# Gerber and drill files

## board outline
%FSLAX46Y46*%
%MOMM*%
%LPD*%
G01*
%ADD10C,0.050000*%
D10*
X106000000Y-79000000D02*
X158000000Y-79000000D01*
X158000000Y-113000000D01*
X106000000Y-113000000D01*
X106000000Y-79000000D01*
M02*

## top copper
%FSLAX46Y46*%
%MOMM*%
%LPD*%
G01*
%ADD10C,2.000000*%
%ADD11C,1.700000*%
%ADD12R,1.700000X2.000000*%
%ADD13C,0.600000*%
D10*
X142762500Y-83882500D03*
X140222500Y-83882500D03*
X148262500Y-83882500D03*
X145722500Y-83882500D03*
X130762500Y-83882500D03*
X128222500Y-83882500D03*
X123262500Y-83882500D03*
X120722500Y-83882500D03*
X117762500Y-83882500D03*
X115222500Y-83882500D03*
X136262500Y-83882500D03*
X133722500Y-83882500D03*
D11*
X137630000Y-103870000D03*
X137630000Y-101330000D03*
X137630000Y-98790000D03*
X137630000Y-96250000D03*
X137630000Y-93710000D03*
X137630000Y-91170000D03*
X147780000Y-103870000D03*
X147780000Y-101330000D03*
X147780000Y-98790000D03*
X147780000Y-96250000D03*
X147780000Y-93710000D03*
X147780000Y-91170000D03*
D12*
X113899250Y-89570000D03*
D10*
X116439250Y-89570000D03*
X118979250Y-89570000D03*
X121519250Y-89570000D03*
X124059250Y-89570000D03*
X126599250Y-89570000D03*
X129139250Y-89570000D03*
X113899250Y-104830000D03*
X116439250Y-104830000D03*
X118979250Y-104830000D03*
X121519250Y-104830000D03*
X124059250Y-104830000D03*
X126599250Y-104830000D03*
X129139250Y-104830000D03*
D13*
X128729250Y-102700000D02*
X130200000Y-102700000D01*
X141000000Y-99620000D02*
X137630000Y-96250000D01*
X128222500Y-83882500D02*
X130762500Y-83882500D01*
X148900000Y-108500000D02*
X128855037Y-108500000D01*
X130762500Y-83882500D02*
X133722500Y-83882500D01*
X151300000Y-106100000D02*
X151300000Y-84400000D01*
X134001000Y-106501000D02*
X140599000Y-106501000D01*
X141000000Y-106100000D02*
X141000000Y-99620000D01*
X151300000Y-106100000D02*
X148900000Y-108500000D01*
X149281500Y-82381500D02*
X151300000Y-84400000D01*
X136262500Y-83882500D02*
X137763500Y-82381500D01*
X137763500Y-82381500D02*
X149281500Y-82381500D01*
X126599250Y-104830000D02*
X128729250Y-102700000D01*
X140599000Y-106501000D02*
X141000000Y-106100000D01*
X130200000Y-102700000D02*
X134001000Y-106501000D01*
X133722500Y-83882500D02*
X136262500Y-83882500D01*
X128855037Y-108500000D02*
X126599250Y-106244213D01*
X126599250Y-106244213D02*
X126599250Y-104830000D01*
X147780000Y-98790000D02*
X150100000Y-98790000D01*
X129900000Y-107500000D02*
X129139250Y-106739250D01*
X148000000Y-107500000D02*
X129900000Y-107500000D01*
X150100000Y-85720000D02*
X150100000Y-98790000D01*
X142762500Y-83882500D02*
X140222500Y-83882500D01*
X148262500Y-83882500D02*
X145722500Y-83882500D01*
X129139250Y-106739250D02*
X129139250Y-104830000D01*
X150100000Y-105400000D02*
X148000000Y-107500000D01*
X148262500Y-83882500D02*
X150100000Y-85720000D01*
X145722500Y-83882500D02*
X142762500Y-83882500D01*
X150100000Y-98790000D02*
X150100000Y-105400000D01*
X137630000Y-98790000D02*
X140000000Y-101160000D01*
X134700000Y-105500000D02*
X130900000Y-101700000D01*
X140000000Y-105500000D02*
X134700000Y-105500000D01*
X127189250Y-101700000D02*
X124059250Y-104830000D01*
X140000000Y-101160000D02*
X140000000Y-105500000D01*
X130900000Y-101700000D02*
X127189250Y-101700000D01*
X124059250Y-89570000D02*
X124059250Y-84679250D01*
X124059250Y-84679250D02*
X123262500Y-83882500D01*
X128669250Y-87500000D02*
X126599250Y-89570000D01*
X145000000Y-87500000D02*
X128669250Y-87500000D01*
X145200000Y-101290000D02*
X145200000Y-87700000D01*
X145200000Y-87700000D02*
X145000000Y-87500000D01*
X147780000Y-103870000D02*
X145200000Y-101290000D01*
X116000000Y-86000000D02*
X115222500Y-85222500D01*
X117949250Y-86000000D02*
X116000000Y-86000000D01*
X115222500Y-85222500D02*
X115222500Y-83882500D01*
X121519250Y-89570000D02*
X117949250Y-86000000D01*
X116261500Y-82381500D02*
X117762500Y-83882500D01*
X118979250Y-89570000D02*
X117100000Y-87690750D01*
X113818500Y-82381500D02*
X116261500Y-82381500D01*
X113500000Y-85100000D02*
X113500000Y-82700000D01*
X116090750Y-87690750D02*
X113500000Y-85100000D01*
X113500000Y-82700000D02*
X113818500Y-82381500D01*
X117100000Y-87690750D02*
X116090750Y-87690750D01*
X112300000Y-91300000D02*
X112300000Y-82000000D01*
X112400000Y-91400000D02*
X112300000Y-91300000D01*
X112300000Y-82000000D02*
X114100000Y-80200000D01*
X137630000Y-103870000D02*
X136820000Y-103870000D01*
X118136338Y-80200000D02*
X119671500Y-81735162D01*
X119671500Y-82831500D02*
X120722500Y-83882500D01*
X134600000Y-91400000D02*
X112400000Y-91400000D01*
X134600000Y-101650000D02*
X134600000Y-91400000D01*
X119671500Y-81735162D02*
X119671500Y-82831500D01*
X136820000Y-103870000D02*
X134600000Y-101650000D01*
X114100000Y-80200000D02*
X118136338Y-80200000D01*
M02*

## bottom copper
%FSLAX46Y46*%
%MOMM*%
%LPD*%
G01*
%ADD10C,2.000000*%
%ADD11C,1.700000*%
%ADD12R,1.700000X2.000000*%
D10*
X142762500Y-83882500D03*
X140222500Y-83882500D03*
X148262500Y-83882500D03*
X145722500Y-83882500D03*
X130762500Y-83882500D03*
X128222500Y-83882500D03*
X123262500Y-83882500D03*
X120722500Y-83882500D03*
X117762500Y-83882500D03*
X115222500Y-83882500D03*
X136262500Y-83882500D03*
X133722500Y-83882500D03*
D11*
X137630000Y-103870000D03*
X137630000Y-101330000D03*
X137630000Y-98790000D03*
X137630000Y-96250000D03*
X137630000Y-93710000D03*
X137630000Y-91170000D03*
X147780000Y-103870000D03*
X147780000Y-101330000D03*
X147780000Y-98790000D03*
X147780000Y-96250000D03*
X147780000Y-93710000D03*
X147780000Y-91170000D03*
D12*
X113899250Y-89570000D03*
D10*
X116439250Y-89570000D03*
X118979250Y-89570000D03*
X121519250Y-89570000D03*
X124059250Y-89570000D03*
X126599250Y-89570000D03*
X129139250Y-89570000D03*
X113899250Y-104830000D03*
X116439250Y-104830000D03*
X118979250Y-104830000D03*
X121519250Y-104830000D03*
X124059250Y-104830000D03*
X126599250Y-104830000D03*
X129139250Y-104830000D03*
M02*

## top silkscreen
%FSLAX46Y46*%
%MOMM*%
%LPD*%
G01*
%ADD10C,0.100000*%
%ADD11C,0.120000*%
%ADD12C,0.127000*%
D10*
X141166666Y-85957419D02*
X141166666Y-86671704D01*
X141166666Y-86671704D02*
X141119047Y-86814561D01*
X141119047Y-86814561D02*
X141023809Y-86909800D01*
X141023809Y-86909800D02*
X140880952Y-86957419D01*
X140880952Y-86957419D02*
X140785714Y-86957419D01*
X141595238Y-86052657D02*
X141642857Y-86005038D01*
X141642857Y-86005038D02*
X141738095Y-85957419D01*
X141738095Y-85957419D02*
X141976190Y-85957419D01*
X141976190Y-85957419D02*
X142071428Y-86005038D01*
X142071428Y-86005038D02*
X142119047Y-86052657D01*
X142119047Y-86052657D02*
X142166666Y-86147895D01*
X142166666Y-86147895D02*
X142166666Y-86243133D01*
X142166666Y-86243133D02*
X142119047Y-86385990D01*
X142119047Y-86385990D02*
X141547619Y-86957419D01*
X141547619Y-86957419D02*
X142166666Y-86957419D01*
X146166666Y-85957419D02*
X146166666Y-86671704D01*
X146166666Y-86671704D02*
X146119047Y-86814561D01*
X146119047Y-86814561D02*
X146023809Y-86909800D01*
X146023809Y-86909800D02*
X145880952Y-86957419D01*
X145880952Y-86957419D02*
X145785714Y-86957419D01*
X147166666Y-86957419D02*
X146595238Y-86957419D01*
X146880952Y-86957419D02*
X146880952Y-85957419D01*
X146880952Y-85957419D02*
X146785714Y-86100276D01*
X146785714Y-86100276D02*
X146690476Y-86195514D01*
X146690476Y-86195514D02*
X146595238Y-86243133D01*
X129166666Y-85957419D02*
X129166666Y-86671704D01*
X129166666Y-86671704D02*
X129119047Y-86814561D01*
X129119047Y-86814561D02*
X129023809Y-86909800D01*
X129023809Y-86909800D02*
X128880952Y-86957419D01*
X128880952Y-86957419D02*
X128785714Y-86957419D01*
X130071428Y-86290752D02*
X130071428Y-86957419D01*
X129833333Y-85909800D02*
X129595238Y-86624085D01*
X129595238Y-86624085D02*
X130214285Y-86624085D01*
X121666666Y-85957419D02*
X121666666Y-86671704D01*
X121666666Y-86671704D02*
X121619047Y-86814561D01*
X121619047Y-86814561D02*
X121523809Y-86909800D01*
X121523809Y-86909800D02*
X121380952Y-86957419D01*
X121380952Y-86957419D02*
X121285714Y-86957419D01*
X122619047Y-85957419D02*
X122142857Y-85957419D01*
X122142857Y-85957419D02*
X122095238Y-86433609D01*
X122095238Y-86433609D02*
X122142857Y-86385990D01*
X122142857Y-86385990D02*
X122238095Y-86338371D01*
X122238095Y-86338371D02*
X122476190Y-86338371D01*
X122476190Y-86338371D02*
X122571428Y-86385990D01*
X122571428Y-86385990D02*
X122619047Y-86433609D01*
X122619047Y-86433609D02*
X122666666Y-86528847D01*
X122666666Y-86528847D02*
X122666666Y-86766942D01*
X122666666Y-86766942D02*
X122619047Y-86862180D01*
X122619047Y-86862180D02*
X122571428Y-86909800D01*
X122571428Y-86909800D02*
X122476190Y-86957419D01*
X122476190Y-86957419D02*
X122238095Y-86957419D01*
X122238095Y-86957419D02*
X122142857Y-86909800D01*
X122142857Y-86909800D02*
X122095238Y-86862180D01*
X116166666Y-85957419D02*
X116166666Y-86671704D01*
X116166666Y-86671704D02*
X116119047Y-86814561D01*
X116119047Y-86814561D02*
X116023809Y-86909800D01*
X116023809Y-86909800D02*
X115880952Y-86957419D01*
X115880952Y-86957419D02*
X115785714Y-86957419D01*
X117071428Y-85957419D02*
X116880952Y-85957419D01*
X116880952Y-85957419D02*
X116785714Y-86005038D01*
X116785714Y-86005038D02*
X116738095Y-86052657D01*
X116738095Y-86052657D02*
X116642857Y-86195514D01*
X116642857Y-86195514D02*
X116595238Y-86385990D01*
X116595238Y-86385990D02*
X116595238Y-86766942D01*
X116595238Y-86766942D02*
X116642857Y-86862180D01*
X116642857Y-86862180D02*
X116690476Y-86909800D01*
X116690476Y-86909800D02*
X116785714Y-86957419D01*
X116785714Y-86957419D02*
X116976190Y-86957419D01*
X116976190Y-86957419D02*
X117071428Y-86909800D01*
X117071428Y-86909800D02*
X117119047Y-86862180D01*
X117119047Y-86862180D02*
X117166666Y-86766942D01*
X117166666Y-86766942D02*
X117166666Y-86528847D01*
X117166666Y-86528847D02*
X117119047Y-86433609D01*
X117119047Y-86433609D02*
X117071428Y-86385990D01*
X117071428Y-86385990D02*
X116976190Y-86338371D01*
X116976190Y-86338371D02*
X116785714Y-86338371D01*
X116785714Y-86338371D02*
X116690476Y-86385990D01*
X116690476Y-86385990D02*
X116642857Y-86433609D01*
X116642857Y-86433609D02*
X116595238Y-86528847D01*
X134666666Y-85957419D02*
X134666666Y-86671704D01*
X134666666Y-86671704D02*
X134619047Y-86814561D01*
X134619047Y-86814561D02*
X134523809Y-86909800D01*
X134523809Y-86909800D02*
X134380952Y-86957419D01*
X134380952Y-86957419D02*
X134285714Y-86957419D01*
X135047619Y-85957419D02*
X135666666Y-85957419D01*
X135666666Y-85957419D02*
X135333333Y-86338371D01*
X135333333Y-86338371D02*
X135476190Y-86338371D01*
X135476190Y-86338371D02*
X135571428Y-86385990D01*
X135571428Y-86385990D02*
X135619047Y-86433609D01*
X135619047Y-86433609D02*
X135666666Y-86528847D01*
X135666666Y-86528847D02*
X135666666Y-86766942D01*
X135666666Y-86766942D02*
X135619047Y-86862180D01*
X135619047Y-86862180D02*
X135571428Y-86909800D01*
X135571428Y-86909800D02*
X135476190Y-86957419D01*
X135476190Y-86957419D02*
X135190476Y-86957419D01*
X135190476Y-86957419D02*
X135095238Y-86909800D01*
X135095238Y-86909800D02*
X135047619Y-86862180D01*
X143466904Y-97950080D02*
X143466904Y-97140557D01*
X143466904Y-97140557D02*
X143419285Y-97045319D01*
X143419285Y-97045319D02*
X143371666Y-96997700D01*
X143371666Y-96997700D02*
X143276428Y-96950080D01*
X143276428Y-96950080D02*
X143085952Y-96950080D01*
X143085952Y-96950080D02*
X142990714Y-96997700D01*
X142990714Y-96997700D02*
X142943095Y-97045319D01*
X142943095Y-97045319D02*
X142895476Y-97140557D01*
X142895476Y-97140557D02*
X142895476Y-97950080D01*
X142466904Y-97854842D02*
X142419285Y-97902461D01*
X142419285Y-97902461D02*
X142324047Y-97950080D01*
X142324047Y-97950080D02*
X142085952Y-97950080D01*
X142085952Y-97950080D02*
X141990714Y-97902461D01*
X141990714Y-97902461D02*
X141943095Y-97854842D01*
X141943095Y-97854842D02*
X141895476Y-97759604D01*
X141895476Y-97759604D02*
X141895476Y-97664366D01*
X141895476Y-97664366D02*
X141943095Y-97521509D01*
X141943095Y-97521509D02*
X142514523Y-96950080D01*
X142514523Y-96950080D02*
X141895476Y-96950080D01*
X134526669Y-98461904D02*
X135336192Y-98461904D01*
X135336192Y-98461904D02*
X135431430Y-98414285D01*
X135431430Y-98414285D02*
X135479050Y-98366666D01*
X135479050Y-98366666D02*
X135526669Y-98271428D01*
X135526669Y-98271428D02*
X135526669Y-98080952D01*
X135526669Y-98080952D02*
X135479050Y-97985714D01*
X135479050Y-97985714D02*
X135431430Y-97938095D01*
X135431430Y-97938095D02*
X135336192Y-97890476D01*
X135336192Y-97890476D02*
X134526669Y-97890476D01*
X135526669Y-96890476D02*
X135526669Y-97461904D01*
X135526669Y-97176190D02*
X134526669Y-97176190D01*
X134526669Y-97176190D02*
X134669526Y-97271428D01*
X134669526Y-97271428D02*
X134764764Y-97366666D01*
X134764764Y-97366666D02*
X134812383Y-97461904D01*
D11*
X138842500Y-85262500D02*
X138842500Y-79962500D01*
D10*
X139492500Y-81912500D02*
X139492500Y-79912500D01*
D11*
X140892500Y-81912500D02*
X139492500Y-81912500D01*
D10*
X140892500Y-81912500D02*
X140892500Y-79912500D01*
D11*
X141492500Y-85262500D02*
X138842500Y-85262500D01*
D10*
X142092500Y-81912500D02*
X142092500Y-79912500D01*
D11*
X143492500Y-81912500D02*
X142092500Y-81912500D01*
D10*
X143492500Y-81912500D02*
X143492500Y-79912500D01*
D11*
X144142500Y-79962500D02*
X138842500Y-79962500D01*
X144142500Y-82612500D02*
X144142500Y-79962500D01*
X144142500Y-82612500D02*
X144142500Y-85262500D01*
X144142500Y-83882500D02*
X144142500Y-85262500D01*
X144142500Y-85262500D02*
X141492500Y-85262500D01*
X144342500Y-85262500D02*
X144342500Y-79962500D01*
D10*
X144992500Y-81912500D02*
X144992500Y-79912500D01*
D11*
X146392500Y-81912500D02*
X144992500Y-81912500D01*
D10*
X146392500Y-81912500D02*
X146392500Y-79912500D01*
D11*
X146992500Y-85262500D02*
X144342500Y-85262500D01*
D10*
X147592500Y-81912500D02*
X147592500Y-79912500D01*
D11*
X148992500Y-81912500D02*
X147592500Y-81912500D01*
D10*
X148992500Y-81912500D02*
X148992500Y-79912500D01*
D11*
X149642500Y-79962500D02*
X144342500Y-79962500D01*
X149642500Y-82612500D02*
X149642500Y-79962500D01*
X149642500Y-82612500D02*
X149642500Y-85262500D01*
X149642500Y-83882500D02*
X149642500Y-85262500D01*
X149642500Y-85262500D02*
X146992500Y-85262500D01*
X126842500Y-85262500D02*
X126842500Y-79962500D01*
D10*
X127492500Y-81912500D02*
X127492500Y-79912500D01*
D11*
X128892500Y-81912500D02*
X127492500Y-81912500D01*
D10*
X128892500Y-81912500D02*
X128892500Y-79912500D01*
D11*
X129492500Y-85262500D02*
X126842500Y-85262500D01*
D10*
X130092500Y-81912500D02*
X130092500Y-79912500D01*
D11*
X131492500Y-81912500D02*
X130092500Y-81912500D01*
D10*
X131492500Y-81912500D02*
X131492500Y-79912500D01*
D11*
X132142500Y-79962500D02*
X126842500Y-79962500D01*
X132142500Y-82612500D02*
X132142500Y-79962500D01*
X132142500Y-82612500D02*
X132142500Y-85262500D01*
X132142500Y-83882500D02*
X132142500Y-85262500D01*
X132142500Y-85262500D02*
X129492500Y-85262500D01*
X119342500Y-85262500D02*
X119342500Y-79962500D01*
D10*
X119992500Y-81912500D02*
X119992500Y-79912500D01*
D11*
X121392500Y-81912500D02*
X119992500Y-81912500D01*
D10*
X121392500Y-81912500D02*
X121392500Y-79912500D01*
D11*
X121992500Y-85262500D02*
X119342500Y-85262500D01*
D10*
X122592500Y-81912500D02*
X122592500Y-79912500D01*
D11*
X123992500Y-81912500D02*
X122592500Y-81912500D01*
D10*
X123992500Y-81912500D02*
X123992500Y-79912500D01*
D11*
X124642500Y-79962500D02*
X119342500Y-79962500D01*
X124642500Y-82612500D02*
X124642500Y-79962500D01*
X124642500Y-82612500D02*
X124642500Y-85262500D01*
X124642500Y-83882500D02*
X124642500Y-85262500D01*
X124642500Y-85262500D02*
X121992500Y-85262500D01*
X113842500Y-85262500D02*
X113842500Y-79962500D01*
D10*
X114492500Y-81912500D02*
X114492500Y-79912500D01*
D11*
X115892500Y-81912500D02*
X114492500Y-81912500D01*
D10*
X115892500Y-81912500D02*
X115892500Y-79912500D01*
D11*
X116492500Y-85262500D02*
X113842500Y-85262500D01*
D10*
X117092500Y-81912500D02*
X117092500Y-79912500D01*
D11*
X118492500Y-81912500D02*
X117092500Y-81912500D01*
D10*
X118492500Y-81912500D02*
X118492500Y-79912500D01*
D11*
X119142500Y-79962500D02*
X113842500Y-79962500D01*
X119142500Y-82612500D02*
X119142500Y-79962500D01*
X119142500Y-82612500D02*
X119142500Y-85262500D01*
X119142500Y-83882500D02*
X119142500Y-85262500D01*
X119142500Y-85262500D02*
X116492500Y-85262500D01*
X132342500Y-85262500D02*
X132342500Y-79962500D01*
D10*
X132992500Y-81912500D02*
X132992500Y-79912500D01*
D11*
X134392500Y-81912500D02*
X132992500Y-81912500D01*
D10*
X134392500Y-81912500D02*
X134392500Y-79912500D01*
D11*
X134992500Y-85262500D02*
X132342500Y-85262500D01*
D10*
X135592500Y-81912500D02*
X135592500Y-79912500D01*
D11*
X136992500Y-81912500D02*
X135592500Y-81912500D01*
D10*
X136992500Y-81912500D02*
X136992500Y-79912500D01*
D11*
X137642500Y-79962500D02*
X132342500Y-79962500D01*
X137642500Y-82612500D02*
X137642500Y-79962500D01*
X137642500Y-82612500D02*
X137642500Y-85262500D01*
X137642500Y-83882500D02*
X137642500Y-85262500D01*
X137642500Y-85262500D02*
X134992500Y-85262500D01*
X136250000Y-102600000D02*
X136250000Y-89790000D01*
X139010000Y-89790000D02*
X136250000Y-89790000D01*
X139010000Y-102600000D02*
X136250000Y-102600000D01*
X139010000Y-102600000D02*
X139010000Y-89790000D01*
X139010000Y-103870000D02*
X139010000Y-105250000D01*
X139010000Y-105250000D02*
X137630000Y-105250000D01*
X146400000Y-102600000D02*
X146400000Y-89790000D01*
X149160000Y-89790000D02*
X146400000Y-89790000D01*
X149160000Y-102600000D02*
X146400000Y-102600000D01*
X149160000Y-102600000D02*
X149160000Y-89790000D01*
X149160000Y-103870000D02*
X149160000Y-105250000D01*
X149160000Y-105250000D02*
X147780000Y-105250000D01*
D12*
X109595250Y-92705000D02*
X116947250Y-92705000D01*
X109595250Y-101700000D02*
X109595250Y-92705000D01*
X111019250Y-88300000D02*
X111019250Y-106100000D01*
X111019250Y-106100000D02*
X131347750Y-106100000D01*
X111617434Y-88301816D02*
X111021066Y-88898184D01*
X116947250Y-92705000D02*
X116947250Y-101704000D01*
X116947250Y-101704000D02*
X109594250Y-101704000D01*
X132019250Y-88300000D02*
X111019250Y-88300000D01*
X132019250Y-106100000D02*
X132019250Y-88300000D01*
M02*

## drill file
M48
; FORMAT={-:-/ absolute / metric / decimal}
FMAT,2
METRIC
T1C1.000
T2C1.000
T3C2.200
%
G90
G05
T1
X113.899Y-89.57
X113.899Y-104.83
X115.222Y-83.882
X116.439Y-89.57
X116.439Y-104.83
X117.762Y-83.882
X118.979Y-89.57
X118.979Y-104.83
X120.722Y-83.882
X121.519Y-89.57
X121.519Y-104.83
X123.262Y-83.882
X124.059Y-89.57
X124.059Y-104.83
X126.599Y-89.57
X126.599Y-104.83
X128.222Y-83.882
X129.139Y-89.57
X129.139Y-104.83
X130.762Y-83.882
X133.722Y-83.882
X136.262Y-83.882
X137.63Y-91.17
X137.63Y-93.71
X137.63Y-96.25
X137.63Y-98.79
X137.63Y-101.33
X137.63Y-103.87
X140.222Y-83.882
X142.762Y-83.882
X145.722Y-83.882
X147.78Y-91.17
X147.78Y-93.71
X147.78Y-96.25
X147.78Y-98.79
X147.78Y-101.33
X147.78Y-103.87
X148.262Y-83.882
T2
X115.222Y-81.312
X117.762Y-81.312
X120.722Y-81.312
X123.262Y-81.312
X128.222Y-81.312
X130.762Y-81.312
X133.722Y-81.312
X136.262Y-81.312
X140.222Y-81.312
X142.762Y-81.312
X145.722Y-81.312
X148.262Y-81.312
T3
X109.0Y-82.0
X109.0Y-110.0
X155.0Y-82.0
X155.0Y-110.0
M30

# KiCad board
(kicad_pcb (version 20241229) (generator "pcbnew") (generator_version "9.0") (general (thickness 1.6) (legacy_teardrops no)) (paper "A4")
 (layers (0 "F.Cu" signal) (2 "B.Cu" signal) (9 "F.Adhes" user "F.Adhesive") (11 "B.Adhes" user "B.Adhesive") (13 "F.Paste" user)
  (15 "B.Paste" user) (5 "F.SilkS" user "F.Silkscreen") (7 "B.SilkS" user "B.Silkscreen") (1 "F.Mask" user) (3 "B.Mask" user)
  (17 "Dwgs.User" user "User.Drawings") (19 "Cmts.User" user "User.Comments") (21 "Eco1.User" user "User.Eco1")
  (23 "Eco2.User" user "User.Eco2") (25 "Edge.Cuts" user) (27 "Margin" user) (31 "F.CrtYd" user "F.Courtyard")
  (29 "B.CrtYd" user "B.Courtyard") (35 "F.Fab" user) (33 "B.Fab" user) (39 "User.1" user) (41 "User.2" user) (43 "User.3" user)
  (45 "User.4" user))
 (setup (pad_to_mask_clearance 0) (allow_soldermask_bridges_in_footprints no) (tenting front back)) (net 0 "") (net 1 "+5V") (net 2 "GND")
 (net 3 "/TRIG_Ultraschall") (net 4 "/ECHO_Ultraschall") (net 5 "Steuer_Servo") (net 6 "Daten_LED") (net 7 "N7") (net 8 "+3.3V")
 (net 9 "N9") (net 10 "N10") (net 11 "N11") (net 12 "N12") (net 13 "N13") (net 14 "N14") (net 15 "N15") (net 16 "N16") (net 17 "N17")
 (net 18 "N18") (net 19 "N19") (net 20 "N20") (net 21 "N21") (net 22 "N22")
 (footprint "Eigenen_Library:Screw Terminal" (layer "F.Cu") (at 141.4925 79.9125 180)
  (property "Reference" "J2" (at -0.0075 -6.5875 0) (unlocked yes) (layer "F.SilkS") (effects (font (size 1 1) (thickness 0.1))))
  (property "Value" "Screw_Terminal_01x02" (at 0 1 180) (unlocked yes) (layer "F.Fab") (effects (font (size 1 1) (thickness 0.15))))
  (fp_line (start 2.65 -5.35) (end 2.65 -0.05) (stroke (width 0.12) (type solid)) (layer "F.SilkS"))
  (fp_line (start 2 -2) (end 2 0) (stroke (width 0.1) (type default)) (layer "F.SilkS"))
  (fp_line (start 0.6 -2) (end 2 -2) (stroke (width 0.12) (type solid)) (layer "F.SilkS"))
  (fp_line (start 0.6 -2) (end 0.6 0) (stroke (width 0.1) (type default)) (layer "F.SilkS"))
  (fp_line (start 0 -5.35) (end 2.65 -5.35) (stroke (width 0.12) (type solid)) (layer "F.SilkS"))
  (fp_line (start -0.6 -2) (end -0.6 0) (stroke (width 0.1) (type default)) (layer "F.SilkS"))
  (fp_line (start -2 -2) (end -0.6 -2) (stroke (width 0.12) (type solid)) (layer "F.SilkS"))
  (fp_line (start -2 -2) (end -2 0) (stroke (width 0.1) (type default)) (layer "F.SilkS"))
  (fp_line (start -2.65 -0.05) (end 2.65 -0.05) (stroke (width 0.12) (type solid)) (layer "F.SilkS"))
  (fp_line (start -2.65 -2.7) (end -2.65 -0.05) (stroke (width 0.12) (type solid)) (layer "F.SilkS"))
  (fp_line (start -2.65 -2.7) (end -2.65 -5.35) (stroke (width 0.12) (type solid)) (layer "F.SilkS"))
  (fp_line (start -2.65 -3.97) (end -2.65 -5.35) (stroke (width 0.12) (type solid)) (layer "F.SilkS"))
  (fp_line (start -2.65 -5.35) (end 0 -5.35) (stroke (width 0.12) (type solid)) (layer "F.SilkS"))
  (pad "" np_thru_hole circle (at -1.27 -1.4 270) (size 1 1) (drill 1) (layers "*.Mask"))
  (pad "" np_thru_hole circle (at 1.27 -1.4 180) (size 1 1) (drill 1) (layers "*.Mask"))
  (pad "1" thru_hole circle (at -1.27 -3.97 180) (size 2 2) (drill 1) (layers "*.Cu" "*.Mask") (remove_unused_layers no) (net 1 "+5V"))
  (pad "2" thru_hole circle (at 1.27 -3.97 180) (size 2 2) (drill 1) (layers "*.Cu" "*.Mask") (remove_unused_layers no) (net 1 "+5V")))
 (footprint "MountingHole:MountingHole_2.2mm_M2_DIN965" (layer "F.Cu") (at 155 110)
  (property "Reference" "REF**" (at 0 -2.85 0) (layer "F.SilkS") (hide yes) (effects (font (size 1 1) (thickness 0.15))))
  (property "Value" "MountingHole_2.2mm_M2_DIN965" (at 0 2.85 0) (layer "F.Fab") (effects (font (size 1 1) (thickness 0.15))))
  (pad "" np_thru_hole circle (at 0 0) (size 2.2 2.2) (drill 2.2) (layers "*.Cu" "*.Mask")))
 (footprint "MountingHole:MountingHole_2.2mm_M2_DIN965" (layer "F.Cu") (at 155 82)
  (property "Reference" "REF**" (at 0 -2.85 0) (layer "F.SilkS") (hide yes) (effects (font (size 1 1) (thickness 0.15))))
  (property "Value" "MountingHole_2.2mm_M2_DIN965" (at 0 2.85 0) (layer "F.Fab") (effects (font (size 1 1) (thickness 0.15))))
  (pad "" np_thru_hole circle (at 0 0) (size 2.2 2.2) (drill 2.2) (layers "*.Cu" "*.Mask")))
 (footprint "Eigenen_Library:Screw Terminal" (layer "F.Cu") (at 146.9925 79.9125 180)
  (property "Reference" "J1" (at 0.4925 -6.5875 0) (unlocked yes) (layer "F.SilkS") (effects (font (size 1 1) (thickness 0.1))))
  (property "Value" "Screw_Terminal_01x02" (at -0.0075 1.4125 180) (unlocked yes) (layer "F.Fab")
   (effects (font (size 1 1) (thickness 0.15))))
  (fp_line (start 2.65 -5.35) (end 2.65 -0.05) (stroke (width 0.12) (type solid)) (layer "F.SilkS"))
  (fp_line (start 2 -2) (end 2 0) (stroke (width 0.1) (type default)) (layer "F.SilkS"))
  (fp_line (start 0.6 -2) (end 2 -2) (stroke (width 0.12) (type solid)) (layer "F.SilkS"))
  (fp_line (start 0.6 -2) (end 0.6 0) (stroke (width 0.1) (type default)) (layer "F.SilkS"))
  (fp_line (start 0 -5.35) (end 2.65 -5.35) (stroke (width 0.12) (type solid)) (layer "F.SilkS"))
  (fp_line (start -0.6 -2) (end -0.6 0) (stroke (width 0.1) (type default)) (layer "F.SilkS"))
  (fp_line (start -2 -2) (end -0.6 -2) (stroke (width 0.12) (type solid)) (layer "F.SilkS"))
  (fp_line (start -2 -2) (end -2 0) (stroke (width 0.1) (type default)) (layer "F.SilkS"))
  (fp_line (start -2.65 -0.05) (end 2.65 -0.05) (stroke (width 0.12) (type solid)) (layer "F.SilkS"))
  (fp_line (start -2.65 -2.7) (end -2.65 -0.05) (stroke (width 0.12) (type solid)) (layer "F.SilkS"))
  (fp_line (start -2.65 -2.7) (end -2.65 -5.35) (stroke (width 0.12) (type solid)) (layer "F.SilkS"))
  (fp_line (start -2.65 -3.97) (end -2.65 -5.35) (stroke (width 0.12) (type solid)) (layer "F.SilkS"))
  (fp_line (start -2.65 -5.35) (end 0 -5.35) (stroke (width 0.12) (type solid)) (layer "F.SilkS"))
  (pad "" np_thru_hole circle (at -1.27 -1.4 270) (size 1 1) (drill 1) (layers "*.Mask"))
  (pad "" np_thru_hole circle (at 1.27 -1.4 180) (size 1 1) (drill 1) (layers "*.Mask"))
  (pad "1" thru_hole circle (at -1.27 -3.97 180) (size 2 2) (drill 1) (layers "*.Cu" "*.Mask") (remove_unused_layers no) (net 1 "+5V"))
  (pad "2" thru_hole circle (at 1.27 -3.97 180) (size 2 2) (drill 1) (layers "*.Cu" "*.Mask") (remove_unused_layers no) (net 1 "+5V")))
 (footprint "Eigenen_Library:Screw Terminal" (layer "F.Cu") (at 129.4925 79.9125 180)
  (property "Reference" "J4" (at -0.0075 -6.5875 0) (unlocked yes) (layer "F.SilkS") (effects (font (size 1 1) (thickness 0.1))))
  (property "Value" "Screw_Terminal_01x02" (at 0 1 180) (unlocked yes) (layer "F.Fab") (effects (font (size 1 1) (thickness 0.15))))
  (fp_line (start 2.65 -5.35) (end 2.65 -0.05) (stroke (width 0.12) (type solid)) (layer "F.SilkS"))
  (fp_line (start 2 -2) (end 2 0) (stroke (width 0.1) (type default)) (layer "F.SilkS"))
  (fp_line (start 0.6 -2) (end 2 -2) (stroke (width 0.12) (type solid)) (layer "F.SilkS"))
  (fp_line (start 0.6 -2) (end 0.6 0) (stroke (width 0.1) (type default)) (layer "F.SilkS"))
  (fp_line (start 0 -5.35) (end 2.65 -5.35) (stroke (width 0.12) (type solid)) (layer "F.SilkS"))
  (fp_line (start -0.6 -2) (end -0.6 0) (stroke (width 0.1) (type default)) (layer "F.SilkS"))
  (fp_line (start -2 -2) (end -0.6 -2) (stroke (width 0.12) (type solid)) (layer "F.SilkS"))
  (fp_line (start -2 -2) (end -2 0) (stroke (width 0.1) (type default)) (layer "F.SilkS"))
  (fp_line (start -2.65 -0.05) (end 2.65 -0.05) (stroke (width 0.12) (type solid)) (layer "F.SilkS"))
  (fp_line (start -2.65 -2.7) (end -2.65 -0.05) (stroke (width 0.12) (type solid)) (layer "F.SilkS"))
  (fp_line (start -2.65 -2.7) (end -2.65 -5.35) (stroke (width 0.12) (type solid)) (layer "F.SilkS"))
  (fp_line (start -2.65 -3.97) (end -2.65 -5.35) (stroke (width 0.12) (type solid)) (layer "F.SilkS"))
  (fp_line (start -2.65 -5.35) (end 0 -5.35) (stroke (width 0.12) (type solid)) (layer "F.SilkS"))
  (pad "" np_thru_hole circle (at -1.27 -1.4 270) (size 1 1) (drill 1) (layers "*.Mask"))
  (pad "" np_thru_hole circle (at 1.27 -1.4 180) (size 1 1) (drill 1) (layers "*.Mask"))
  (pad "1" thru_hole circle (at -1.27 -3.97 180) (size 2 2) (drill 1) (layers "*.Cu" "*.Mask") (remove_unused_layers no) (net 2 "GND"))
  (pad "2" thru_hole circle (at 1.27 -3.97 180) (size 2 2) (drill 1) (layers "*.Cu" "*.Mask") (remove_unused_layers no) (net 2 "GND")))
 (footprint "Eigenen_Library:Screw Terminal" (layer "F.Cu") (at 121.9925 79.9125 180)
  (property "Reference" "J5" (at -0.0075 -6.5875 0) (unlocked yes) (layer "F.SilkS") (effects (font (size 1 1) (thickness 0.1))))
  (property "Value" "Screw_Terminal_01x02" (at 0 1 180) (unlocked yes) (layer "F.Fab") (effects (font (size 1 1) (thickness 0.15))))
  (fp_line (start 2.65 -5.35) (end 2.65 -0.05) (stroke (width 0.12) (type solid)) (layer "F.SilkS"))
  (fp_line (start 2 -2) (end 2 0) (stroke (width 0.1) (type default)) (layer "F.SilkS"))
  (fp_line (start 0.6 -2) (end 2 -2) (stroke (width 0.12) (type solid)) (layer "F.SilkS"))
  (fp_line (start 0.6 -2) (end 0.6 0) (stroke (width 0.1) (type default)) (layer "F.SilkS"))
  (fp_line (start 0 -5.35) (end 2.65 -5.35) (stroke (width 0.12) (type solid)) (layer "F.SilkS"))
  (fp_line (start -0.6 -2) (end -0.6 0) (stroke (width 0.1) (type default)) (layer "F.SilkS"))
  (fp_line (start -2 -2) (end -0.6 -2) (stroke (width 0.12) (type solid)) (layer "F.SilkS"))
  (fp_line (start -2 -2) (end -2 0) (stroke (width 0.1) (type default)) (layer "F.SilkS"))
  (fp_line (start -2.65 -0.05) (end 2.65 -0.05) (stroke (width 0.12) (type solid)) (layer "F.SilkS"))
  (fp_line (start -2.65 -2.7) (end -2.65 -0.05) (stroke (width 0.12) (type solid)) (layer "F.SilkS"))
  (fp_line (start -2.65 -2.7) (end -2.65 -5.35) (stroke (width 0.12) (type solid)) (layer "F.SilkS"))
  (fp_line (start -2.65 -3.97) (end -2.65 -5.35) (stroke (width 0.12) (type solid)) (layer "F.SilkS"))
  (fp_line (start -2.65 -5.35) (end 0 -5.35) (stroke (width 0.12) (type solid)) (layer "F.SilkS"))
  (pad "" np_thru_hole circle (at -1.27 -1.4 270) (size 1 1) (drill 1) (layers "*.Mask"))
  (pad "" np_thru_hole circle (at 1.27 -1.4 180) (size 1 1) (drill 1) (layers "*.Mask"))
  (pad "1" thru_hole circle (at -1.27 -3.97 180) (size 2 2) (drill 1) (layers "*.Cu" "*.Mask") (remove_unused_layers no)
   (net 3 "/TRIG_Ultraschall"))
  (pad "2" thru_hole circle (at 1.27 -3.97 180) (size 2 2) (drill 1) (layers "*.Cu" "*.Mask") (remove_unused_layers no)
   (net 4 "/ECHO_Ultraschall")))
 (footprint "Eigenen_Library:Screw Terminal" (layer "F.Cu") (at 116.4925 79.9125 180)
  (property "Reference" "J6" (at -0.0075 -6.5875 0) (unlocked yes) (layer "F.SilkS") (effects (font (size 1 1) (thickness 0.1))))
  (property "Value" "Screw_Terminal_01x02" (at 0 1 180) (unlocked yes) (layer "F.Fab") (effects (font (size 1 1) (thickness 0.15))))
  (fp_line (start 2.65 -5.35) (end 2.65 -0.05) (stroke (width 0.12) (type solid)) (layer "F.SilkS"))
  (fp_line (start 2 -2) (end 2 0) (stroke (width 0.1) (type default)) (layer "F.SilkS"))
  (fp_line (start 0.6 -2) (end 2 -2) (stroke (width 0.12) (type solid)) (layer "F.SilkS"))
  (fp_line (start 0.6 -2) (end 0.6 0) (stroke (width 0.1) (type default)) (layer "F.SilkS"))
  (fp_line (start 0 -5.35) (end 2.65 -5.35) (stroke (width 0.12) (type solid)) (layer "F.SilkS"))
  (fp_line (start -0.6 -2) (end -0.6 0) (stroke (width 0.1) (type default)) (layer "F.SilkS"))
  (fp_line (start -2 -2) (end -0.6 -2) (stroke (width 0.12) (type solid)) (layer "F.SilkS"))
  (fp_line (start -2 -2) (end -2 0) (stroke (width 0.1) (type default)) (layer "F.SilkS"))
  (fp_line (start -2.65 -0.05) (end 2.65 -0.05) (stroke (width 0.12) (type solid)) (layer "F.SilkS"))
  (fp_line (start -2.65 -2.7) (end -2.65 -0.05) (stroke (width 0.12) (type solid)) (layer "F.SilkS"))
  (fp_line (start -2.65 -2.7) (end -2.65 -5.35) (stroke (width 0.12) (type solid)) (layer "F.SilkS"))
  (fp_line (start -2.65 -3.97) (end -2.65 -5.35) (stroke (width 0.12) (type solid)) (layer "F.SilkS"))
  (fp_line (start -2.65 -5.35) (end 0 -5.35) (stroke (width 0.12) (type solid)) (layer "F.SilkS"))
  (pad "" np_thru_hole circle (at -1.27 -1.4 270) (size 1 1) (drill 1) (layers "*.Mask"))
  (pad "" np_thru_hole circle (at 1.27 -1.4 180) (size 1 1) (drill 1) (layers "*.Mask"))
  (pad "1" thru_hole circle (at -1.27 -3.97 180) (size 2 2) (drill 1) (layers "*.Cu" "*.Mask") (remove_unused_layers no)
   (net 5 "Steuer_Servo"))
  (pad "2" thru_hole circle (at 1.27 -3.97 180) (size 2 2) (drill 1) (layers "*.Cu" "*.Mask") (remove_unused_layers no) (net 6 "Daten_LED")))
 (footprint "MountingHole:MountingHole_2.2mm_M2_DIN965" (layer "F.Cu") (at 109 110)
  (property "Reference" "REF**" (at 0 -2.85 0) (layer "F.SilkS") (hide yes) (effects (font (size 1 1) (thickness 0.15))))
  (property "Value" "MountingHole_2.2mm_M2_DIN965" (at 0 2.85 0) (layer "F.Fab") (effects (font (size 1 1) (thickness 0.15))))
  (pad "" np_thru_hole circle (at 0 0) (size 2.2 2.2) (drill 2.2) (layers "*.Cu" "*.Mask")))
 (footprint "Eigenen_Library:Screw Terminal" (layer "F.Cu") (at 134.9925 79.9125 180)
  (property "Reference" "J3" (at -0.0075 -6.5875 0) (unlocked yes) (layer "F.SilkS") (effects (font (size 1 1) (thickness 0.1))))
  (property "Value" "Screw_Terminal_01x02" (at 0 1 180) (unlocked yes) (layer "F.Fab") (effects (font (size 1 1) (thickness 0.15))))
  (fp_line (start 2.65 -5.35) (end 2.65 -0.05) (stroke (width 0.12) (type solid)) (layer "F.SilkS"))
  (fp_line (start 2 -2) (end 2 0) (stroke (width 0.1) (type default)) (layer "F.SilkS"))
  (fp_line (start 0.6 -2) (end 2 -2) (stroke (width 0.12) (type solid)) (layer "F.SilkS"))
  (fp_line (start 0.6 -2) (end 0.6 0) (stroke (width 0.1) (type default)) (layer "F.SilkS"))
  (fp_line (start 0 -5.35) (end 2.65 -5.35) (stroke (width 0.12) (type solid)) (layer "F.SilkS"))
  (fp_line (start -0.6 -2) (end -0.6 0) (stroke (width 0.1) (type default)) (layer "F.SilkS"))
  (fp_line (start -2 -2) (end -0.6 -2) (stroke (width 0.12) (type solid)) (layer "F.SilkS"))
  (fp_line (start -2 -2) (end -2 0) (stroke (width 0.1) (type default)) (layer "F.SilkS"))
  (fp_line (start -2.65 -0.05) (end 2.65 -0.05) (stroke (width 0.12) (type solid)) (layer "F.SilkS"))
  (fp_line (start -2.65 -2.7) (end -2.65 -0.05) (stroke (width 0.12) (type solid)) (layer "F.SilkS"))
  (fp_line (start -2.65 -2.7) (end -2.65 -5.35) (stroke (width 0.12) (type solid)) (layer "F.SilkS"))
  (fp_line (start -2.65 -3.97) (end -2.65 -5.35) (stroke (width 0.12) (type solid)) (layer "F.SilkS"))
  (fp_line (start -2.65 -5.35) (end 0 -5.35) (stroke (width 0.12) (type solid)) (layer "F.SilkS"))
  (pad "" np_thru_hole circle (at -1.27 -1.4 270) (size 1 1) (drill 1) (layers "*.Mask"))
  (pad "" np_thru_hole circle (at 1.27 -1.4 180) (size 1 1) (drill 1) (layers "*.Mask"))
  (pad "1" thru_hole circle (at -1.27 -3.97 180) (size 2 2) (drill 1) (layers "*.Cu" "*.Mask") (remove_unused_layers no) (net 2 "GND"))
  (pad "2" thru_hole circle (at 1.27 -3.97 180) (size 2 2) (drill 1) (layers "*.Cu" "*.Mask") (remove_unused_layers no) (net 2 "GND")))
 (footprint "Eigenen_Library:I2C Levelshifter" (layer "F.Cu") (at 142.8 89.4 180)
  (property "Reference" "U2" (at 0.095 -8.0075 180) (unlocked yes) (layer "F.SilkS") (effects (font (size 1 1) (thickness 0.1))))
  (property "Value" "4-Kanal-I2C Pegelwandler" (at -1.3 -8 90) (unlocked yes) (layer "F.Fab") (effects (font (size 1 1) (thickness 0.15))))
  (fp_line (start 6.55 -13.2) (end 6.55 -0.39) (stroke (width 0.12) (type solid)) (layer "F.SilkS"))
  (fp_line (start 3.79 -0.39) (end 6.55 -0.39) (stroke (width 0.12) (type solid)) (layer "F.SilkS"))
  (fp_line (start 3.79 -13.2) (end 6.55 -13.2) (stroke (width 0.12) (type solid)) (layer "F.SilkS"))
  (fp_line (start 3.79 -13.2) (end 3.79 -0.39) (stroke (width 0.12) (type solid)) (layer "F.SilkS"))
  (fp_line (start 3.79 -14.47) (end 3.79 -15.85) (stroke (width 0.12) (type solid)) (layer "F.SilkS"))
  (fp_line (start 3.79 -15.85) (end 5.17 -15.85) (stroke (width 0.12) (type solid)) (layer "F.SilkS"))
  (fp_line (start -3.6 -13.2) (end -3.6 -0.39) (stroke (width 0.12) (type solid)) (layer "F.SilkS"))
  (fp_line (start -6.36 -0.39) (end -3.6 -0.39) (stroke (width 0.12) (type solid)) (layer "F.SilkS"))
  (fp_line (start -6.36 -13.2) (end -3.6 -13.2) (stroke (width 0.12) (type solid)) (layer "F.SilkS"))
  (fp_line (start -6.36 -13.2) (end -6.36 -0.39) (stroke (width 0.12) (type solid)) (layer "F.SilkS"))
  (fp_line (start -6.36 -14.47) (end -6.36 -15.85) (stroke (width 0.12) (type solid)) (layer "F.SilkS"))
  (fp_line (start -6.36 -15.85) (end -4.98 -15.85) (stroke (width 0.12) (type solid)) (layer "F.SilkS"))
  (pad "1" thru_hole circle (at 5.17 -14.47 180) (size 1.7 1.7) (drill 1) (layers "*.Cu" "*.Mask") (remove_unused_layers no)
   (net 4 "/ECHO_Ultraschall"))
  (pad "2" thru_hole circle (at 5.17 -11.93 180) (size 1.7 1.7) (drill 1) (layers "*.Cu" "*.Mask") (remove_unused_layers no) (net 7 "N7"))
  (pad "3" thru_hole circle (at 5.17 -9.39 180) (size 1.7 1.7) (drill 1) (layers "*.Cu" "*.Mask") (remove_unused_layers no) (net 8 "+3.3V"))
  (pad "4" thru_hole circle (at 5.17 -6.85 180) (size 1.7 1.7) (drill 1) (layers "*.Cu" "*.Mask") (remove_unused_layers no) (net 2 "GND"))
  (pad "5" thru_hole circle (at 5.17 -4.31 180) (size 1.7 1.7) (drill 1) (layers "*.Cu" "*.Mask") (remove_unused_layers no) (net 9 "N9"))
  (pad "6" thru_hole circle (at 5.17 -1.77 180) (size 1.7 1.7) (drill 1) (layers "*.Cu" "*.Mask") (remove_unused_layers no) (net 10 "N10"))
  (pad "7" thru_hole circle (at -4.98 -14.47 180) (size 1.7 1.7) (drill 1) (layers "*.Cu" "*.Mask") (remove_unused_layers no) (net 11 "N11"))
  (pad "8" thru_hole circle (at -4.98 -11.93 180) (size 1.7 1.7) (drill 1) (layers "*.Cu" "*.Mask") (remove_unused_layers no) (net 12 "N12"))
  (pad "9" thru_hole circle (at -4.98 -9.39 180) (size 1.7 1.7) (drill 1) (layers "*.Cu" "*.Mask") (remove_unused_layers no) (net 1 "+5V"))
  (pad "10" thru_hole circle (at -4.98 -6.85 180) (size 1.7 1.7) (drill 1) (layers "*.Cu" "*.Mask") (remove_unused_layers no) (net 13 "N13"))
  (pad "11" thru_hole circle (at -4.98 -4.31 180) (size 1.7 1.7) (drill 1) (layers "*.Cu" "*.Mask") (remove_unused_layers no) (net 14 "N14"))
  (pad "12" thru_hole circle (at -4.98 -1.77 180) (size 1.7 1.7) (drill 1) (layers "*.Cu" "*.Mask") (remove_unused_layers no) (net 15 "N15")))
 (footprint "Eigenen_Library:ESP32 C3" (layer "F.Cu") (at 132.01925 97.2 90)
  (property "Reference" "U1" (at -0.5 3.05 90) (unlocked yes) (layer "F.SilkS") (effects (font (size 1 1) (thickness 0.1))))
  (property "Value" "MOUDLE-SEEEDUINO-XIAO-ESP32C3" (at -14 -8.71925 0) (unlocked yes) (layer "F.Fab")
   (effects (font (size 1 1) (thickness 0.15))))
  (fp_line (start 4.495 -22.424) (end 4.495 -15.072) (stroke (width 0.127) (type solid)) (layer "F.SilkS"))
  (fp_line (start -4.5 -22.424) (end 4.495 -22.424) (stroke (width 0.127) (type solid)) (layer "F.SilkS"))
  (fp_line (start 8.9 -21) (end -8.9 -21) (stroke (width 0.127) (type solid)) (layer "F.SilkS"))
  (fp_line (start -8.9 -21) (end -8.9 -0.6715) (stroke (width 0.127) (type solid)) (layer "F.SilkS"))
  (fp_line (start 8.898184 -20.401816) (end 8.301816 -20.998184) (stroke (width 0.127) (type solid)) (layer "F.SilkS"))
  (fp_line (start 4.495 -15.072) (end -4.504 -15.072) (stroke (width 0.127) (type solid)) (layer "F.SilkS"))
  (fp_line (start -4.504 -15.072) (end -4.504 -22.425) (stroke (width 0.127) (type solid)) (layer "F.SilkS"))
  (fp_line (start 8.9 0) (end 8.9 -21) (stroke (width 0.127) (type solid)) (layer "F.SilkS"))
  (fp_line (start -8.9 0) (end 8.9 0) (stroke (width 0.127) (type solid)) (layer "F.SilkS"))
  (pad "1" thru_hole rect (at 7.63 -18.12 90) (size 2 1.7) (drill 1) (layers "*.Cu" "*.Mask") (remove_unused_layers no) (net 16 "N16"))
  (pad "2" thru_hole circle (at 7.63 -15.58 90) (size 2 2) (drill 1) (layers "*.Cu" "*.Mask") (remove_unused_layers no) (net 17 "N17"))
  (pad "3" thru_hole circle (at 7.63 -13.04 90) (size 2 2) (drill 1) (layers "*.Cu" "*.Mask") (remove_unused_layers no)
   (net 5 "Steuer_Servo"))
  (pad "4" thru_hole circle (at 7.63 -10.5 90) (size 2 2) (drill 1) (layers "*.Cu" "*.Mask") (remove_unused_layers no) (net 6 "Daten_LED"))
  (pad "5" thru_hole circle (at 7.63 -7.96 90) (size 2 2) (drill 1) (layers "*.Cu" "*.Mask") (remove_unused_layers no)
   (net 3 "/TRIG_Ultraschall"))
  (pad "6" thru_hole circle (at 7.63 -5.42 90) (size 2 2) (drill 1) (layers "*.Cu" "*.Mask") (remove_unused_layers no) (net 11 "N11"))
  (pad "7" thru_hole circle (at 7.63 -2.88 90) (size 2 2) (drill 1) (layers "*.Cu" "*.Mask") (remove_unused_layers no) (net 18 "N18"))
  (pad "8" thru_hole circle (at -7.63 -18.12 90) (size 2 2) (drill 1) (layers "*.Cu" "*.Mask") (remove_unused_layers no) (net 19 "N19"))
  (pad "9" thru_hole circle (at -7.63 -15.58 90) (size 2 2) (drill 1) (layers "*.Cu" "*.Mask") (remove_unused_layers no) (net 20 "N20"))
  (pad "10" thru_hole circle (at -7.63 -13.04 90) (size 2 2) (drill 1) (layers "*.Cu" "*.Mask") (remove_unused_layers no) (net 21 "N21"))
  (pad "11" thru_hole circle (at -7.63 -10.5 90) (size 2 2) (drill 1) (layers "*.Cu" "*.Mask") (remove_unused_layers no) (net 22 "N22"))
  (pad "12" thru_hole circle (at -7.63 -7.96 90) (size 2 2) (drill 1) (layers "*.Cu" "*.Mask") (remove_unused_layers no) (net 8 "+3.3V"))
  (pad "13" thru_hole circle (at -7.63 -5.42 90) (size 2 2) (drill 1) (layers "*.Cu" "*.Mask") (remove_unused_layers no) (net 2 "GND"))
  (pad "14" thru_hole circle (at -7.63 -2.88 90) (size 2 2) (drill 1) (layers "*.Cu" "*.Mask") (remove_unused_layers no) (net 1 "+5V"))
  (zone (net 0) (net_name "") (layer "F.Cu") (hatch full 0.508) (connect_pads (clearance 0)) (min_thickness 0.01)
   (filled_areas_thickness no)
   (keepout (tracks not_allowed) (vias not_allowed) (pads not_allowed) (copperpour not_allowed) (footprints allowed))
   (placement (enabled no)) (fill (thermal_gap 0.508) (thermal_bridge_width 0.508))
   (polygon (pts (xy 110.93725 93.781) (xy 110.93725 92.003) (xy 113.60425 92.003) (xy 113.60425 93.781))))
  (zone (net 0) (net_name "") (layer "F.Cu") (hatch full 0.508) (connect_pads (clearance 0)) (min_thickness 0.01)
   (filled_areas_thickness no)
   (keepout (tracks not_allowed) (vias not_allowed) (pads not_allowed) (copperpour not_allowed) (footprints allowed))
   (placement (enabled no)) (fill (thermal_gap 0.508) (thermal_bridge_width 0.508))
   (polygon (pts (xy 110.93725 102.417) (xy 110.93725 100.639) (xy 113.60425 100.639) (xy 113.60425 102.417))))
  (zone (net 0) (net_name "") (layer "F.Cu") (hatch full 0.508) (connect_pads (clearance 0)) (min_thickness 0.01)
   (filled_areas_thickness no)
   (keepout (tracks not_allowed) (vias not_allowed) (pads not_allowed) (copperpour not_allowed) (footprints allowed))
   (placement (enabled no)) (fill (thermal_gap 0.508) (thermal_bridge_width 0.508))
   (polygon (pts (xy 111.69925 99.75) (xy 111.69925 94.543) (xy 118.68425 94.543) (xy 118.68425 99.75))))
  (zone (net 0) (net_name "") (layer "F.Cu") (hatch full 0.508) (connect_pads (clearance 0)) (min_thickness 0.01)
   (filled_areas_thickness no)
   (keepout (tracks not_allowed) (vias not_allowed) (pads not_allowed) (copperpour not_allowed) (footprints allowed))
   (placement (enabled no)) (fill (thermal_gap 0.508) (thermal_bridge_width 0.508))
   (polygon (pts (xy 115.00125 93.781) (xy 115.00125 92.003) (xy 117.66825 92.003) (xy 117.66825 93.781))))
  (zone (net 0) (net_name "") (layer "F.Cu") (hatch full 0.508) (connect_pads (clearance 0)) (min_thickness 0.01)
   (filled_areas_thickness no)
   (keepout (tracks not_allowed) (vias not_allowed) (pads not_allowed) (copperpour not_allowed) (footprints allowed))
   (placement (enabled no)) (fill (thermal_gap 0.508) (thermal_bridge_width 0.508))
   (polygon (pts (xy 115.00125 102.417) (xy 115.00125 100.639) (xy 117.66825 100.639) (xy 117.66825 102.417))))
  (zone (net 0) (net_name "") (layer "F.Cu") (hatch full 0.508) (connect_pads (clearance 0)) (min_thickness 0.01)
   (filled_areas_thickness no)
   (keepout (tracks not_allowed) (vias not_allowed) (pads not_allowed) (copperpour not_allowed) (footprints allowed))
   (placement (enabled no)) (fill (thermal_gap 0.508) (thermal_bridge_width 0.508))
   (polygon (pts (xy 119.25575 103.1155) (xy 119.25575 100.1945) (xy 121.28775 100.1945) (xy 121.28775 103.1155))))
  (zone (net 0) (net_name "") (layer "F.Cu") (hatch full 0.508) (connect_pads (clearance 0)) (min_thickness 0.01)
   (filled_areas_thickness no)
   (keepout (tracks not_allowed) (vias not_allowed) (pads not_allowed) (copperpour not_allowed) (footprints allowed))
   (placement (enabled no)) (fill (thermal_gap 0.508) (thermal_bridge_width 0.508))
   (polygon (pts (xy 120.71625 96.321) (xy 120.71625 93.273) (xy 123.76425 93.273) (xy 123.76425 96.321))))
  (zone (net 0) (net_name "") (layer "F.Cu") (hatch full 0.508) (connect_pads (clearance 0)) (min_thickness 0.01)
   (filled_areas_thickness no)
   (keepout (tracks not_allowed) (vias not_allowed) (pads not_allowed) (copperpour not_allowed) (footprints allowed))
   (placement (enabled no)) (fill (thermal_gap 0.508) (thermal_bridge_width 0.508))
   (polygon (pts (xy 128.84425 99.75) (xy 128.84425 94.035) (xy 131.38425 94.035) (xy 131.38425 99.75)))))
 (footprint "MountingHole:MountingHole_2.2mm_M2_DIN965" (layer "F.Cu") (at 109 82)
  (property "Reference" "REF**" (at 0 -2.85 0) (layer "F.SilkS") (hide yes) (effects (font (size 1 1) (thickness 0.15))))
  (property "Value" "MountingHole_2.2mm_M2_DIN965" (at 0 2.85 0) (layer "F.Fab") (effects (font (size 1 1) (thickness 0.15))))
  (pad "" np_thru_hole circle (at 0 0) (size 2.2 2.2) (drill 2.2) (layers "*.Cu" "*.Mask")))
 (gr_rect (start 106 79) (end 158 113) (stroke (width 0.05) (type solid)) (fill no) (layer "Edge.Cuts"))
 (segment (start 128.72925 102.7) (end 130.2 102.7) (width 0.6) (layer "F.Cu") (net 2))
 (segment (start 141 99.62) (end 137.63 96.25) (width 0.6) (layer "F.Cu") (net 2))
 (segment (start 128.2225 83.8825) (end 130.7625 83.8825) (width 0.6) (layer "F.Cu") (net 2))
 (segment (start 148.9 108.5) (end 128.855037 108.5) (width 0.6) (layer "F.Cu") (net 2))
 (segment (start 130.7625 83.8825) (end 133.7225 83.8825) (width 0.6) (layer "F.Cu") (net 2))
 (segment (start 151.3 106.1) (end 151.3 84.4) (width 0.6) (layer "F.Cu") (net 2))
 (segment (start 134.001 106.501) (end 140.599 106.501) (width 0.6) (layer "F.Cu") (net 2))
 (segment (start 141 106.1) (end 141 99.62) (width 0.6) (layer "F.Cu") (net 2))
 (segment (start 151.3 106.1) (end 148.9 108.5) (width 0.6) (layer "F.Cu") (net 2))
 (segment (start 149.2815 82.3815) (end 151.3 84.4) (width 0.6) (layer "F.Cu") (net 2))
 (segment (start 136.2625 83.8825) (end 137.7635 82.3815) (width 0.6) (layer "F.Cu") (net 2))
 (segment (start 137.7635 82.3815) (end 149.2815 82.3815) (width 0.6) (layer "F.Cu") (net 2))
 (segment (start 126.59925 104.83) (end 128.72925 102.7) (width 0.6) (layer "F.Cu") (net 2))
 (segment (start 140.599 106.501) (end 141 106.1) (width 0.6) (layer "F.Cu") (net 2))
 (segment (start 130.2 102.7) (end 134.001 106.501) (width 0.6) (layer "F.Cu") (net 2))
 (segment (start 133.7225 83.8825) (end 136.2625 83.8825) (width 0.6) (layer "F.Cu") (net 2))
 (segment (start 128.855037 108.5) (end 126.59925 106.244213) (width 0.6) (layer "F.Cu") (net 2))
 (segment (start 126.59925 106.244213) (end 126.59925 104.83) (width 0.6) (layer "F.Cu") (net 2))
 (segment (start 147.78 98.79) (end 150.1 98.79) (width 0.6) (layer "F.Cu") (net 1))
 (segment (start 129.9 107.5) (end 129.13925 106.73925) (width 0.6) (layer "F.Cu") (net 1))
 (segment (start 148 107.5) (end 129.9 107.5) (width 0.6) (layer "F.Cu") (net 1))
 (segment (start 150.1 85.72) (end 150.1 98.79) (width 0.6) (layer "F.Cu") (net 1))
 (segment (start 142.7625 83.8825) (end 140.2225 83.8825) (width 0.6) (layer "F.Cu") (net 1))
 (segment (start 148.2625 83.8825) (end 145.7225 83.8825) (width 0.6) (layer "F.Cu") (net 1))
 (segment (start 129.13925 106.73925) (end 129.13925 104.83) (width 0.6) (layer "F.Cu") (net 1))
 (segment (start 150.1 105.4) (end 148 107.5) (width 0.6) (layer "F.Cu") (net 1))
 (segment (start 148.2625 83.8825) (end 150.1 85.72) (width 0.6) (layer "F.Cu") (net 1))
 (segment (start 145.7225 83.8825) (end 142.7625 83.8825) (width 0.6) (layer "F.Cu") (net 1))
 (segment (start 150.1 98.79) (end 150.1 105.4) (width 0.6) (layer "F.Cu") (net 1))
 (segment (start 137.63 98.79) (end 140 101.16) (width 0.6) (layer "F.Cu") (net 8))
 (segment (start 134.7 105.5) (end 130.9 101.7) (width 0.6) (layer "F.Cu") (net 8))
 (segment (start 140 105.5) (end 134.7 105.5) (width 0.6) (layer "F.Cu") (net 8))
 (segment (start 127.18925 101.7) (end 124.05925 104.83) (width 0.6) (layer "F.Cu") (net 8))
 (segment (start 140 101.16) (end 140 105.5) (width 0.6) (layer "F.Cu") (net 8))
 (segment (start 130.9 101.7) (end 127.18925 101.7) (width 0.6) (layer "F.Cu") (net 8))
 (segment (start 124.05925 89.57) (end 124.05925 84.67925) (width 0.6) (layer "F.Cu") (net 3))
 (segment (start 124.05925 84.67925) (end 123.2625 83.8825) (width 0.6) (layer "F.Cu") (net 3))
 (segment (start 128.66925 87.5) (end 126.59925 89.57) (width 0.6) (layer "F.Cu") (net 11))
 (segment (start 145 87.5) (end 128.66925 87.5) (width 0.6) (layer "F.Cu") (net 11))
 (segment (start 145.2 101.29) (end 145.2 87.7) (width 0.6) (layer "F.Cu") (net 11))
 (segment (start 145.2 87.7) (end 145 87.5) (width 0.6) (layer "F.Cu") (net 11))
 (segment (start 147.78 103.87) (end 145.2 101.29) (width 0.6) (layer "F.Cu") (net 11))
 (segment (start 116 86) (end 115.2225 85.2225) (width 0.6) (layer "F.Cu") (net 6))
 (segment (start 117.94925 86) (end 116 86) (width 0.6) (layer "F.Cu") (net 6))
 (segment (start 115.2225 85.2225) (end 115.2225 83.8825) (width 0.6) (layer "F.Cu") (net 6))
 (segment (start 121.51925 89.57) (end 117.94925 86) (width 0.6) (layer "F.Cu") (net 6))
 (segment (start 116.2615 82.3815) (end 117.7625 83.8825) (width 0.6) (layer "F.Cu") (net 5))
 (segment (start 118.97925 89.57) (end 117.1 87.69075) (width 0.6) (layer "F.Cu") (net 5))
 (segment (start 113.8185 82.3815) (end 116.2615 82.3815) (width 0.6) (layer "F.Cu") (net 5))
 (segment (start 113.5 85.1) (end 113.5 82.7) (width 0.6) (layer "F.Cu") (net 5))
 (segment (start 116.09075 87.69075) (end 113.5 85.1) (width 0.6) (layer "F.Cu") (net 5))
 (segment (start 113.5 82.7) (end 113.8185 82.3815) (width 0.6) (layer "F.Cu") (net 5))
 (segment (start 117.1 87.69075) (end 116.09075 87.69075) (width 0.6) (layer "F.Cu") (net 5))
 (segment (start 112.3 91.3) (end 112.3 82) (width 0.6) (layer "F.Cu") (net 4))
 (segment (start 112.4 91.4) (end 112.3 91.3) (width 0.6) (layer "F.Cu") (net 4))
 (segment (start 112.3 82) (end 114.1 80.2) (width 0.6) (layer "F.Cu") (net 4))
 (segment (start 137.63 103.87) (end 136.82 103.87) (width 0.6) (layer "F.Cu") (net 4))
 (segment (start 118.136338 80.2) (end 119.6715 81.735162) (width 0.6) (layer "F.Cu") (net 4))
 (segment (start 119.6715 82.8315) (end 120.7225 83.8825) (width 0.6) (layer "F.Cu") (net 4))
 (segment (start 134.6 91.4) (end 112.4 91.4) (width 0.6) (layer "F.Cu") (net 4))
 (segment (start 134.6 101.65) (end 134.6 91.4) (width 0.6) (layer "F.Cu") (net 4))
 (segment (start 119.6715 81.735162) (end 119.6715 82.8315) (width 0.6) (layer "F.Cu") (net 4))
 (segment (start 136.82 103.87) (end 134.6 101.65) (width 0.6) (layer "F.Cu") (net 4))
 (segment (start 114.1 80.2) (end 118.136338 80.2) (width 0.6) (layer "F.Cu") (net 4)))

